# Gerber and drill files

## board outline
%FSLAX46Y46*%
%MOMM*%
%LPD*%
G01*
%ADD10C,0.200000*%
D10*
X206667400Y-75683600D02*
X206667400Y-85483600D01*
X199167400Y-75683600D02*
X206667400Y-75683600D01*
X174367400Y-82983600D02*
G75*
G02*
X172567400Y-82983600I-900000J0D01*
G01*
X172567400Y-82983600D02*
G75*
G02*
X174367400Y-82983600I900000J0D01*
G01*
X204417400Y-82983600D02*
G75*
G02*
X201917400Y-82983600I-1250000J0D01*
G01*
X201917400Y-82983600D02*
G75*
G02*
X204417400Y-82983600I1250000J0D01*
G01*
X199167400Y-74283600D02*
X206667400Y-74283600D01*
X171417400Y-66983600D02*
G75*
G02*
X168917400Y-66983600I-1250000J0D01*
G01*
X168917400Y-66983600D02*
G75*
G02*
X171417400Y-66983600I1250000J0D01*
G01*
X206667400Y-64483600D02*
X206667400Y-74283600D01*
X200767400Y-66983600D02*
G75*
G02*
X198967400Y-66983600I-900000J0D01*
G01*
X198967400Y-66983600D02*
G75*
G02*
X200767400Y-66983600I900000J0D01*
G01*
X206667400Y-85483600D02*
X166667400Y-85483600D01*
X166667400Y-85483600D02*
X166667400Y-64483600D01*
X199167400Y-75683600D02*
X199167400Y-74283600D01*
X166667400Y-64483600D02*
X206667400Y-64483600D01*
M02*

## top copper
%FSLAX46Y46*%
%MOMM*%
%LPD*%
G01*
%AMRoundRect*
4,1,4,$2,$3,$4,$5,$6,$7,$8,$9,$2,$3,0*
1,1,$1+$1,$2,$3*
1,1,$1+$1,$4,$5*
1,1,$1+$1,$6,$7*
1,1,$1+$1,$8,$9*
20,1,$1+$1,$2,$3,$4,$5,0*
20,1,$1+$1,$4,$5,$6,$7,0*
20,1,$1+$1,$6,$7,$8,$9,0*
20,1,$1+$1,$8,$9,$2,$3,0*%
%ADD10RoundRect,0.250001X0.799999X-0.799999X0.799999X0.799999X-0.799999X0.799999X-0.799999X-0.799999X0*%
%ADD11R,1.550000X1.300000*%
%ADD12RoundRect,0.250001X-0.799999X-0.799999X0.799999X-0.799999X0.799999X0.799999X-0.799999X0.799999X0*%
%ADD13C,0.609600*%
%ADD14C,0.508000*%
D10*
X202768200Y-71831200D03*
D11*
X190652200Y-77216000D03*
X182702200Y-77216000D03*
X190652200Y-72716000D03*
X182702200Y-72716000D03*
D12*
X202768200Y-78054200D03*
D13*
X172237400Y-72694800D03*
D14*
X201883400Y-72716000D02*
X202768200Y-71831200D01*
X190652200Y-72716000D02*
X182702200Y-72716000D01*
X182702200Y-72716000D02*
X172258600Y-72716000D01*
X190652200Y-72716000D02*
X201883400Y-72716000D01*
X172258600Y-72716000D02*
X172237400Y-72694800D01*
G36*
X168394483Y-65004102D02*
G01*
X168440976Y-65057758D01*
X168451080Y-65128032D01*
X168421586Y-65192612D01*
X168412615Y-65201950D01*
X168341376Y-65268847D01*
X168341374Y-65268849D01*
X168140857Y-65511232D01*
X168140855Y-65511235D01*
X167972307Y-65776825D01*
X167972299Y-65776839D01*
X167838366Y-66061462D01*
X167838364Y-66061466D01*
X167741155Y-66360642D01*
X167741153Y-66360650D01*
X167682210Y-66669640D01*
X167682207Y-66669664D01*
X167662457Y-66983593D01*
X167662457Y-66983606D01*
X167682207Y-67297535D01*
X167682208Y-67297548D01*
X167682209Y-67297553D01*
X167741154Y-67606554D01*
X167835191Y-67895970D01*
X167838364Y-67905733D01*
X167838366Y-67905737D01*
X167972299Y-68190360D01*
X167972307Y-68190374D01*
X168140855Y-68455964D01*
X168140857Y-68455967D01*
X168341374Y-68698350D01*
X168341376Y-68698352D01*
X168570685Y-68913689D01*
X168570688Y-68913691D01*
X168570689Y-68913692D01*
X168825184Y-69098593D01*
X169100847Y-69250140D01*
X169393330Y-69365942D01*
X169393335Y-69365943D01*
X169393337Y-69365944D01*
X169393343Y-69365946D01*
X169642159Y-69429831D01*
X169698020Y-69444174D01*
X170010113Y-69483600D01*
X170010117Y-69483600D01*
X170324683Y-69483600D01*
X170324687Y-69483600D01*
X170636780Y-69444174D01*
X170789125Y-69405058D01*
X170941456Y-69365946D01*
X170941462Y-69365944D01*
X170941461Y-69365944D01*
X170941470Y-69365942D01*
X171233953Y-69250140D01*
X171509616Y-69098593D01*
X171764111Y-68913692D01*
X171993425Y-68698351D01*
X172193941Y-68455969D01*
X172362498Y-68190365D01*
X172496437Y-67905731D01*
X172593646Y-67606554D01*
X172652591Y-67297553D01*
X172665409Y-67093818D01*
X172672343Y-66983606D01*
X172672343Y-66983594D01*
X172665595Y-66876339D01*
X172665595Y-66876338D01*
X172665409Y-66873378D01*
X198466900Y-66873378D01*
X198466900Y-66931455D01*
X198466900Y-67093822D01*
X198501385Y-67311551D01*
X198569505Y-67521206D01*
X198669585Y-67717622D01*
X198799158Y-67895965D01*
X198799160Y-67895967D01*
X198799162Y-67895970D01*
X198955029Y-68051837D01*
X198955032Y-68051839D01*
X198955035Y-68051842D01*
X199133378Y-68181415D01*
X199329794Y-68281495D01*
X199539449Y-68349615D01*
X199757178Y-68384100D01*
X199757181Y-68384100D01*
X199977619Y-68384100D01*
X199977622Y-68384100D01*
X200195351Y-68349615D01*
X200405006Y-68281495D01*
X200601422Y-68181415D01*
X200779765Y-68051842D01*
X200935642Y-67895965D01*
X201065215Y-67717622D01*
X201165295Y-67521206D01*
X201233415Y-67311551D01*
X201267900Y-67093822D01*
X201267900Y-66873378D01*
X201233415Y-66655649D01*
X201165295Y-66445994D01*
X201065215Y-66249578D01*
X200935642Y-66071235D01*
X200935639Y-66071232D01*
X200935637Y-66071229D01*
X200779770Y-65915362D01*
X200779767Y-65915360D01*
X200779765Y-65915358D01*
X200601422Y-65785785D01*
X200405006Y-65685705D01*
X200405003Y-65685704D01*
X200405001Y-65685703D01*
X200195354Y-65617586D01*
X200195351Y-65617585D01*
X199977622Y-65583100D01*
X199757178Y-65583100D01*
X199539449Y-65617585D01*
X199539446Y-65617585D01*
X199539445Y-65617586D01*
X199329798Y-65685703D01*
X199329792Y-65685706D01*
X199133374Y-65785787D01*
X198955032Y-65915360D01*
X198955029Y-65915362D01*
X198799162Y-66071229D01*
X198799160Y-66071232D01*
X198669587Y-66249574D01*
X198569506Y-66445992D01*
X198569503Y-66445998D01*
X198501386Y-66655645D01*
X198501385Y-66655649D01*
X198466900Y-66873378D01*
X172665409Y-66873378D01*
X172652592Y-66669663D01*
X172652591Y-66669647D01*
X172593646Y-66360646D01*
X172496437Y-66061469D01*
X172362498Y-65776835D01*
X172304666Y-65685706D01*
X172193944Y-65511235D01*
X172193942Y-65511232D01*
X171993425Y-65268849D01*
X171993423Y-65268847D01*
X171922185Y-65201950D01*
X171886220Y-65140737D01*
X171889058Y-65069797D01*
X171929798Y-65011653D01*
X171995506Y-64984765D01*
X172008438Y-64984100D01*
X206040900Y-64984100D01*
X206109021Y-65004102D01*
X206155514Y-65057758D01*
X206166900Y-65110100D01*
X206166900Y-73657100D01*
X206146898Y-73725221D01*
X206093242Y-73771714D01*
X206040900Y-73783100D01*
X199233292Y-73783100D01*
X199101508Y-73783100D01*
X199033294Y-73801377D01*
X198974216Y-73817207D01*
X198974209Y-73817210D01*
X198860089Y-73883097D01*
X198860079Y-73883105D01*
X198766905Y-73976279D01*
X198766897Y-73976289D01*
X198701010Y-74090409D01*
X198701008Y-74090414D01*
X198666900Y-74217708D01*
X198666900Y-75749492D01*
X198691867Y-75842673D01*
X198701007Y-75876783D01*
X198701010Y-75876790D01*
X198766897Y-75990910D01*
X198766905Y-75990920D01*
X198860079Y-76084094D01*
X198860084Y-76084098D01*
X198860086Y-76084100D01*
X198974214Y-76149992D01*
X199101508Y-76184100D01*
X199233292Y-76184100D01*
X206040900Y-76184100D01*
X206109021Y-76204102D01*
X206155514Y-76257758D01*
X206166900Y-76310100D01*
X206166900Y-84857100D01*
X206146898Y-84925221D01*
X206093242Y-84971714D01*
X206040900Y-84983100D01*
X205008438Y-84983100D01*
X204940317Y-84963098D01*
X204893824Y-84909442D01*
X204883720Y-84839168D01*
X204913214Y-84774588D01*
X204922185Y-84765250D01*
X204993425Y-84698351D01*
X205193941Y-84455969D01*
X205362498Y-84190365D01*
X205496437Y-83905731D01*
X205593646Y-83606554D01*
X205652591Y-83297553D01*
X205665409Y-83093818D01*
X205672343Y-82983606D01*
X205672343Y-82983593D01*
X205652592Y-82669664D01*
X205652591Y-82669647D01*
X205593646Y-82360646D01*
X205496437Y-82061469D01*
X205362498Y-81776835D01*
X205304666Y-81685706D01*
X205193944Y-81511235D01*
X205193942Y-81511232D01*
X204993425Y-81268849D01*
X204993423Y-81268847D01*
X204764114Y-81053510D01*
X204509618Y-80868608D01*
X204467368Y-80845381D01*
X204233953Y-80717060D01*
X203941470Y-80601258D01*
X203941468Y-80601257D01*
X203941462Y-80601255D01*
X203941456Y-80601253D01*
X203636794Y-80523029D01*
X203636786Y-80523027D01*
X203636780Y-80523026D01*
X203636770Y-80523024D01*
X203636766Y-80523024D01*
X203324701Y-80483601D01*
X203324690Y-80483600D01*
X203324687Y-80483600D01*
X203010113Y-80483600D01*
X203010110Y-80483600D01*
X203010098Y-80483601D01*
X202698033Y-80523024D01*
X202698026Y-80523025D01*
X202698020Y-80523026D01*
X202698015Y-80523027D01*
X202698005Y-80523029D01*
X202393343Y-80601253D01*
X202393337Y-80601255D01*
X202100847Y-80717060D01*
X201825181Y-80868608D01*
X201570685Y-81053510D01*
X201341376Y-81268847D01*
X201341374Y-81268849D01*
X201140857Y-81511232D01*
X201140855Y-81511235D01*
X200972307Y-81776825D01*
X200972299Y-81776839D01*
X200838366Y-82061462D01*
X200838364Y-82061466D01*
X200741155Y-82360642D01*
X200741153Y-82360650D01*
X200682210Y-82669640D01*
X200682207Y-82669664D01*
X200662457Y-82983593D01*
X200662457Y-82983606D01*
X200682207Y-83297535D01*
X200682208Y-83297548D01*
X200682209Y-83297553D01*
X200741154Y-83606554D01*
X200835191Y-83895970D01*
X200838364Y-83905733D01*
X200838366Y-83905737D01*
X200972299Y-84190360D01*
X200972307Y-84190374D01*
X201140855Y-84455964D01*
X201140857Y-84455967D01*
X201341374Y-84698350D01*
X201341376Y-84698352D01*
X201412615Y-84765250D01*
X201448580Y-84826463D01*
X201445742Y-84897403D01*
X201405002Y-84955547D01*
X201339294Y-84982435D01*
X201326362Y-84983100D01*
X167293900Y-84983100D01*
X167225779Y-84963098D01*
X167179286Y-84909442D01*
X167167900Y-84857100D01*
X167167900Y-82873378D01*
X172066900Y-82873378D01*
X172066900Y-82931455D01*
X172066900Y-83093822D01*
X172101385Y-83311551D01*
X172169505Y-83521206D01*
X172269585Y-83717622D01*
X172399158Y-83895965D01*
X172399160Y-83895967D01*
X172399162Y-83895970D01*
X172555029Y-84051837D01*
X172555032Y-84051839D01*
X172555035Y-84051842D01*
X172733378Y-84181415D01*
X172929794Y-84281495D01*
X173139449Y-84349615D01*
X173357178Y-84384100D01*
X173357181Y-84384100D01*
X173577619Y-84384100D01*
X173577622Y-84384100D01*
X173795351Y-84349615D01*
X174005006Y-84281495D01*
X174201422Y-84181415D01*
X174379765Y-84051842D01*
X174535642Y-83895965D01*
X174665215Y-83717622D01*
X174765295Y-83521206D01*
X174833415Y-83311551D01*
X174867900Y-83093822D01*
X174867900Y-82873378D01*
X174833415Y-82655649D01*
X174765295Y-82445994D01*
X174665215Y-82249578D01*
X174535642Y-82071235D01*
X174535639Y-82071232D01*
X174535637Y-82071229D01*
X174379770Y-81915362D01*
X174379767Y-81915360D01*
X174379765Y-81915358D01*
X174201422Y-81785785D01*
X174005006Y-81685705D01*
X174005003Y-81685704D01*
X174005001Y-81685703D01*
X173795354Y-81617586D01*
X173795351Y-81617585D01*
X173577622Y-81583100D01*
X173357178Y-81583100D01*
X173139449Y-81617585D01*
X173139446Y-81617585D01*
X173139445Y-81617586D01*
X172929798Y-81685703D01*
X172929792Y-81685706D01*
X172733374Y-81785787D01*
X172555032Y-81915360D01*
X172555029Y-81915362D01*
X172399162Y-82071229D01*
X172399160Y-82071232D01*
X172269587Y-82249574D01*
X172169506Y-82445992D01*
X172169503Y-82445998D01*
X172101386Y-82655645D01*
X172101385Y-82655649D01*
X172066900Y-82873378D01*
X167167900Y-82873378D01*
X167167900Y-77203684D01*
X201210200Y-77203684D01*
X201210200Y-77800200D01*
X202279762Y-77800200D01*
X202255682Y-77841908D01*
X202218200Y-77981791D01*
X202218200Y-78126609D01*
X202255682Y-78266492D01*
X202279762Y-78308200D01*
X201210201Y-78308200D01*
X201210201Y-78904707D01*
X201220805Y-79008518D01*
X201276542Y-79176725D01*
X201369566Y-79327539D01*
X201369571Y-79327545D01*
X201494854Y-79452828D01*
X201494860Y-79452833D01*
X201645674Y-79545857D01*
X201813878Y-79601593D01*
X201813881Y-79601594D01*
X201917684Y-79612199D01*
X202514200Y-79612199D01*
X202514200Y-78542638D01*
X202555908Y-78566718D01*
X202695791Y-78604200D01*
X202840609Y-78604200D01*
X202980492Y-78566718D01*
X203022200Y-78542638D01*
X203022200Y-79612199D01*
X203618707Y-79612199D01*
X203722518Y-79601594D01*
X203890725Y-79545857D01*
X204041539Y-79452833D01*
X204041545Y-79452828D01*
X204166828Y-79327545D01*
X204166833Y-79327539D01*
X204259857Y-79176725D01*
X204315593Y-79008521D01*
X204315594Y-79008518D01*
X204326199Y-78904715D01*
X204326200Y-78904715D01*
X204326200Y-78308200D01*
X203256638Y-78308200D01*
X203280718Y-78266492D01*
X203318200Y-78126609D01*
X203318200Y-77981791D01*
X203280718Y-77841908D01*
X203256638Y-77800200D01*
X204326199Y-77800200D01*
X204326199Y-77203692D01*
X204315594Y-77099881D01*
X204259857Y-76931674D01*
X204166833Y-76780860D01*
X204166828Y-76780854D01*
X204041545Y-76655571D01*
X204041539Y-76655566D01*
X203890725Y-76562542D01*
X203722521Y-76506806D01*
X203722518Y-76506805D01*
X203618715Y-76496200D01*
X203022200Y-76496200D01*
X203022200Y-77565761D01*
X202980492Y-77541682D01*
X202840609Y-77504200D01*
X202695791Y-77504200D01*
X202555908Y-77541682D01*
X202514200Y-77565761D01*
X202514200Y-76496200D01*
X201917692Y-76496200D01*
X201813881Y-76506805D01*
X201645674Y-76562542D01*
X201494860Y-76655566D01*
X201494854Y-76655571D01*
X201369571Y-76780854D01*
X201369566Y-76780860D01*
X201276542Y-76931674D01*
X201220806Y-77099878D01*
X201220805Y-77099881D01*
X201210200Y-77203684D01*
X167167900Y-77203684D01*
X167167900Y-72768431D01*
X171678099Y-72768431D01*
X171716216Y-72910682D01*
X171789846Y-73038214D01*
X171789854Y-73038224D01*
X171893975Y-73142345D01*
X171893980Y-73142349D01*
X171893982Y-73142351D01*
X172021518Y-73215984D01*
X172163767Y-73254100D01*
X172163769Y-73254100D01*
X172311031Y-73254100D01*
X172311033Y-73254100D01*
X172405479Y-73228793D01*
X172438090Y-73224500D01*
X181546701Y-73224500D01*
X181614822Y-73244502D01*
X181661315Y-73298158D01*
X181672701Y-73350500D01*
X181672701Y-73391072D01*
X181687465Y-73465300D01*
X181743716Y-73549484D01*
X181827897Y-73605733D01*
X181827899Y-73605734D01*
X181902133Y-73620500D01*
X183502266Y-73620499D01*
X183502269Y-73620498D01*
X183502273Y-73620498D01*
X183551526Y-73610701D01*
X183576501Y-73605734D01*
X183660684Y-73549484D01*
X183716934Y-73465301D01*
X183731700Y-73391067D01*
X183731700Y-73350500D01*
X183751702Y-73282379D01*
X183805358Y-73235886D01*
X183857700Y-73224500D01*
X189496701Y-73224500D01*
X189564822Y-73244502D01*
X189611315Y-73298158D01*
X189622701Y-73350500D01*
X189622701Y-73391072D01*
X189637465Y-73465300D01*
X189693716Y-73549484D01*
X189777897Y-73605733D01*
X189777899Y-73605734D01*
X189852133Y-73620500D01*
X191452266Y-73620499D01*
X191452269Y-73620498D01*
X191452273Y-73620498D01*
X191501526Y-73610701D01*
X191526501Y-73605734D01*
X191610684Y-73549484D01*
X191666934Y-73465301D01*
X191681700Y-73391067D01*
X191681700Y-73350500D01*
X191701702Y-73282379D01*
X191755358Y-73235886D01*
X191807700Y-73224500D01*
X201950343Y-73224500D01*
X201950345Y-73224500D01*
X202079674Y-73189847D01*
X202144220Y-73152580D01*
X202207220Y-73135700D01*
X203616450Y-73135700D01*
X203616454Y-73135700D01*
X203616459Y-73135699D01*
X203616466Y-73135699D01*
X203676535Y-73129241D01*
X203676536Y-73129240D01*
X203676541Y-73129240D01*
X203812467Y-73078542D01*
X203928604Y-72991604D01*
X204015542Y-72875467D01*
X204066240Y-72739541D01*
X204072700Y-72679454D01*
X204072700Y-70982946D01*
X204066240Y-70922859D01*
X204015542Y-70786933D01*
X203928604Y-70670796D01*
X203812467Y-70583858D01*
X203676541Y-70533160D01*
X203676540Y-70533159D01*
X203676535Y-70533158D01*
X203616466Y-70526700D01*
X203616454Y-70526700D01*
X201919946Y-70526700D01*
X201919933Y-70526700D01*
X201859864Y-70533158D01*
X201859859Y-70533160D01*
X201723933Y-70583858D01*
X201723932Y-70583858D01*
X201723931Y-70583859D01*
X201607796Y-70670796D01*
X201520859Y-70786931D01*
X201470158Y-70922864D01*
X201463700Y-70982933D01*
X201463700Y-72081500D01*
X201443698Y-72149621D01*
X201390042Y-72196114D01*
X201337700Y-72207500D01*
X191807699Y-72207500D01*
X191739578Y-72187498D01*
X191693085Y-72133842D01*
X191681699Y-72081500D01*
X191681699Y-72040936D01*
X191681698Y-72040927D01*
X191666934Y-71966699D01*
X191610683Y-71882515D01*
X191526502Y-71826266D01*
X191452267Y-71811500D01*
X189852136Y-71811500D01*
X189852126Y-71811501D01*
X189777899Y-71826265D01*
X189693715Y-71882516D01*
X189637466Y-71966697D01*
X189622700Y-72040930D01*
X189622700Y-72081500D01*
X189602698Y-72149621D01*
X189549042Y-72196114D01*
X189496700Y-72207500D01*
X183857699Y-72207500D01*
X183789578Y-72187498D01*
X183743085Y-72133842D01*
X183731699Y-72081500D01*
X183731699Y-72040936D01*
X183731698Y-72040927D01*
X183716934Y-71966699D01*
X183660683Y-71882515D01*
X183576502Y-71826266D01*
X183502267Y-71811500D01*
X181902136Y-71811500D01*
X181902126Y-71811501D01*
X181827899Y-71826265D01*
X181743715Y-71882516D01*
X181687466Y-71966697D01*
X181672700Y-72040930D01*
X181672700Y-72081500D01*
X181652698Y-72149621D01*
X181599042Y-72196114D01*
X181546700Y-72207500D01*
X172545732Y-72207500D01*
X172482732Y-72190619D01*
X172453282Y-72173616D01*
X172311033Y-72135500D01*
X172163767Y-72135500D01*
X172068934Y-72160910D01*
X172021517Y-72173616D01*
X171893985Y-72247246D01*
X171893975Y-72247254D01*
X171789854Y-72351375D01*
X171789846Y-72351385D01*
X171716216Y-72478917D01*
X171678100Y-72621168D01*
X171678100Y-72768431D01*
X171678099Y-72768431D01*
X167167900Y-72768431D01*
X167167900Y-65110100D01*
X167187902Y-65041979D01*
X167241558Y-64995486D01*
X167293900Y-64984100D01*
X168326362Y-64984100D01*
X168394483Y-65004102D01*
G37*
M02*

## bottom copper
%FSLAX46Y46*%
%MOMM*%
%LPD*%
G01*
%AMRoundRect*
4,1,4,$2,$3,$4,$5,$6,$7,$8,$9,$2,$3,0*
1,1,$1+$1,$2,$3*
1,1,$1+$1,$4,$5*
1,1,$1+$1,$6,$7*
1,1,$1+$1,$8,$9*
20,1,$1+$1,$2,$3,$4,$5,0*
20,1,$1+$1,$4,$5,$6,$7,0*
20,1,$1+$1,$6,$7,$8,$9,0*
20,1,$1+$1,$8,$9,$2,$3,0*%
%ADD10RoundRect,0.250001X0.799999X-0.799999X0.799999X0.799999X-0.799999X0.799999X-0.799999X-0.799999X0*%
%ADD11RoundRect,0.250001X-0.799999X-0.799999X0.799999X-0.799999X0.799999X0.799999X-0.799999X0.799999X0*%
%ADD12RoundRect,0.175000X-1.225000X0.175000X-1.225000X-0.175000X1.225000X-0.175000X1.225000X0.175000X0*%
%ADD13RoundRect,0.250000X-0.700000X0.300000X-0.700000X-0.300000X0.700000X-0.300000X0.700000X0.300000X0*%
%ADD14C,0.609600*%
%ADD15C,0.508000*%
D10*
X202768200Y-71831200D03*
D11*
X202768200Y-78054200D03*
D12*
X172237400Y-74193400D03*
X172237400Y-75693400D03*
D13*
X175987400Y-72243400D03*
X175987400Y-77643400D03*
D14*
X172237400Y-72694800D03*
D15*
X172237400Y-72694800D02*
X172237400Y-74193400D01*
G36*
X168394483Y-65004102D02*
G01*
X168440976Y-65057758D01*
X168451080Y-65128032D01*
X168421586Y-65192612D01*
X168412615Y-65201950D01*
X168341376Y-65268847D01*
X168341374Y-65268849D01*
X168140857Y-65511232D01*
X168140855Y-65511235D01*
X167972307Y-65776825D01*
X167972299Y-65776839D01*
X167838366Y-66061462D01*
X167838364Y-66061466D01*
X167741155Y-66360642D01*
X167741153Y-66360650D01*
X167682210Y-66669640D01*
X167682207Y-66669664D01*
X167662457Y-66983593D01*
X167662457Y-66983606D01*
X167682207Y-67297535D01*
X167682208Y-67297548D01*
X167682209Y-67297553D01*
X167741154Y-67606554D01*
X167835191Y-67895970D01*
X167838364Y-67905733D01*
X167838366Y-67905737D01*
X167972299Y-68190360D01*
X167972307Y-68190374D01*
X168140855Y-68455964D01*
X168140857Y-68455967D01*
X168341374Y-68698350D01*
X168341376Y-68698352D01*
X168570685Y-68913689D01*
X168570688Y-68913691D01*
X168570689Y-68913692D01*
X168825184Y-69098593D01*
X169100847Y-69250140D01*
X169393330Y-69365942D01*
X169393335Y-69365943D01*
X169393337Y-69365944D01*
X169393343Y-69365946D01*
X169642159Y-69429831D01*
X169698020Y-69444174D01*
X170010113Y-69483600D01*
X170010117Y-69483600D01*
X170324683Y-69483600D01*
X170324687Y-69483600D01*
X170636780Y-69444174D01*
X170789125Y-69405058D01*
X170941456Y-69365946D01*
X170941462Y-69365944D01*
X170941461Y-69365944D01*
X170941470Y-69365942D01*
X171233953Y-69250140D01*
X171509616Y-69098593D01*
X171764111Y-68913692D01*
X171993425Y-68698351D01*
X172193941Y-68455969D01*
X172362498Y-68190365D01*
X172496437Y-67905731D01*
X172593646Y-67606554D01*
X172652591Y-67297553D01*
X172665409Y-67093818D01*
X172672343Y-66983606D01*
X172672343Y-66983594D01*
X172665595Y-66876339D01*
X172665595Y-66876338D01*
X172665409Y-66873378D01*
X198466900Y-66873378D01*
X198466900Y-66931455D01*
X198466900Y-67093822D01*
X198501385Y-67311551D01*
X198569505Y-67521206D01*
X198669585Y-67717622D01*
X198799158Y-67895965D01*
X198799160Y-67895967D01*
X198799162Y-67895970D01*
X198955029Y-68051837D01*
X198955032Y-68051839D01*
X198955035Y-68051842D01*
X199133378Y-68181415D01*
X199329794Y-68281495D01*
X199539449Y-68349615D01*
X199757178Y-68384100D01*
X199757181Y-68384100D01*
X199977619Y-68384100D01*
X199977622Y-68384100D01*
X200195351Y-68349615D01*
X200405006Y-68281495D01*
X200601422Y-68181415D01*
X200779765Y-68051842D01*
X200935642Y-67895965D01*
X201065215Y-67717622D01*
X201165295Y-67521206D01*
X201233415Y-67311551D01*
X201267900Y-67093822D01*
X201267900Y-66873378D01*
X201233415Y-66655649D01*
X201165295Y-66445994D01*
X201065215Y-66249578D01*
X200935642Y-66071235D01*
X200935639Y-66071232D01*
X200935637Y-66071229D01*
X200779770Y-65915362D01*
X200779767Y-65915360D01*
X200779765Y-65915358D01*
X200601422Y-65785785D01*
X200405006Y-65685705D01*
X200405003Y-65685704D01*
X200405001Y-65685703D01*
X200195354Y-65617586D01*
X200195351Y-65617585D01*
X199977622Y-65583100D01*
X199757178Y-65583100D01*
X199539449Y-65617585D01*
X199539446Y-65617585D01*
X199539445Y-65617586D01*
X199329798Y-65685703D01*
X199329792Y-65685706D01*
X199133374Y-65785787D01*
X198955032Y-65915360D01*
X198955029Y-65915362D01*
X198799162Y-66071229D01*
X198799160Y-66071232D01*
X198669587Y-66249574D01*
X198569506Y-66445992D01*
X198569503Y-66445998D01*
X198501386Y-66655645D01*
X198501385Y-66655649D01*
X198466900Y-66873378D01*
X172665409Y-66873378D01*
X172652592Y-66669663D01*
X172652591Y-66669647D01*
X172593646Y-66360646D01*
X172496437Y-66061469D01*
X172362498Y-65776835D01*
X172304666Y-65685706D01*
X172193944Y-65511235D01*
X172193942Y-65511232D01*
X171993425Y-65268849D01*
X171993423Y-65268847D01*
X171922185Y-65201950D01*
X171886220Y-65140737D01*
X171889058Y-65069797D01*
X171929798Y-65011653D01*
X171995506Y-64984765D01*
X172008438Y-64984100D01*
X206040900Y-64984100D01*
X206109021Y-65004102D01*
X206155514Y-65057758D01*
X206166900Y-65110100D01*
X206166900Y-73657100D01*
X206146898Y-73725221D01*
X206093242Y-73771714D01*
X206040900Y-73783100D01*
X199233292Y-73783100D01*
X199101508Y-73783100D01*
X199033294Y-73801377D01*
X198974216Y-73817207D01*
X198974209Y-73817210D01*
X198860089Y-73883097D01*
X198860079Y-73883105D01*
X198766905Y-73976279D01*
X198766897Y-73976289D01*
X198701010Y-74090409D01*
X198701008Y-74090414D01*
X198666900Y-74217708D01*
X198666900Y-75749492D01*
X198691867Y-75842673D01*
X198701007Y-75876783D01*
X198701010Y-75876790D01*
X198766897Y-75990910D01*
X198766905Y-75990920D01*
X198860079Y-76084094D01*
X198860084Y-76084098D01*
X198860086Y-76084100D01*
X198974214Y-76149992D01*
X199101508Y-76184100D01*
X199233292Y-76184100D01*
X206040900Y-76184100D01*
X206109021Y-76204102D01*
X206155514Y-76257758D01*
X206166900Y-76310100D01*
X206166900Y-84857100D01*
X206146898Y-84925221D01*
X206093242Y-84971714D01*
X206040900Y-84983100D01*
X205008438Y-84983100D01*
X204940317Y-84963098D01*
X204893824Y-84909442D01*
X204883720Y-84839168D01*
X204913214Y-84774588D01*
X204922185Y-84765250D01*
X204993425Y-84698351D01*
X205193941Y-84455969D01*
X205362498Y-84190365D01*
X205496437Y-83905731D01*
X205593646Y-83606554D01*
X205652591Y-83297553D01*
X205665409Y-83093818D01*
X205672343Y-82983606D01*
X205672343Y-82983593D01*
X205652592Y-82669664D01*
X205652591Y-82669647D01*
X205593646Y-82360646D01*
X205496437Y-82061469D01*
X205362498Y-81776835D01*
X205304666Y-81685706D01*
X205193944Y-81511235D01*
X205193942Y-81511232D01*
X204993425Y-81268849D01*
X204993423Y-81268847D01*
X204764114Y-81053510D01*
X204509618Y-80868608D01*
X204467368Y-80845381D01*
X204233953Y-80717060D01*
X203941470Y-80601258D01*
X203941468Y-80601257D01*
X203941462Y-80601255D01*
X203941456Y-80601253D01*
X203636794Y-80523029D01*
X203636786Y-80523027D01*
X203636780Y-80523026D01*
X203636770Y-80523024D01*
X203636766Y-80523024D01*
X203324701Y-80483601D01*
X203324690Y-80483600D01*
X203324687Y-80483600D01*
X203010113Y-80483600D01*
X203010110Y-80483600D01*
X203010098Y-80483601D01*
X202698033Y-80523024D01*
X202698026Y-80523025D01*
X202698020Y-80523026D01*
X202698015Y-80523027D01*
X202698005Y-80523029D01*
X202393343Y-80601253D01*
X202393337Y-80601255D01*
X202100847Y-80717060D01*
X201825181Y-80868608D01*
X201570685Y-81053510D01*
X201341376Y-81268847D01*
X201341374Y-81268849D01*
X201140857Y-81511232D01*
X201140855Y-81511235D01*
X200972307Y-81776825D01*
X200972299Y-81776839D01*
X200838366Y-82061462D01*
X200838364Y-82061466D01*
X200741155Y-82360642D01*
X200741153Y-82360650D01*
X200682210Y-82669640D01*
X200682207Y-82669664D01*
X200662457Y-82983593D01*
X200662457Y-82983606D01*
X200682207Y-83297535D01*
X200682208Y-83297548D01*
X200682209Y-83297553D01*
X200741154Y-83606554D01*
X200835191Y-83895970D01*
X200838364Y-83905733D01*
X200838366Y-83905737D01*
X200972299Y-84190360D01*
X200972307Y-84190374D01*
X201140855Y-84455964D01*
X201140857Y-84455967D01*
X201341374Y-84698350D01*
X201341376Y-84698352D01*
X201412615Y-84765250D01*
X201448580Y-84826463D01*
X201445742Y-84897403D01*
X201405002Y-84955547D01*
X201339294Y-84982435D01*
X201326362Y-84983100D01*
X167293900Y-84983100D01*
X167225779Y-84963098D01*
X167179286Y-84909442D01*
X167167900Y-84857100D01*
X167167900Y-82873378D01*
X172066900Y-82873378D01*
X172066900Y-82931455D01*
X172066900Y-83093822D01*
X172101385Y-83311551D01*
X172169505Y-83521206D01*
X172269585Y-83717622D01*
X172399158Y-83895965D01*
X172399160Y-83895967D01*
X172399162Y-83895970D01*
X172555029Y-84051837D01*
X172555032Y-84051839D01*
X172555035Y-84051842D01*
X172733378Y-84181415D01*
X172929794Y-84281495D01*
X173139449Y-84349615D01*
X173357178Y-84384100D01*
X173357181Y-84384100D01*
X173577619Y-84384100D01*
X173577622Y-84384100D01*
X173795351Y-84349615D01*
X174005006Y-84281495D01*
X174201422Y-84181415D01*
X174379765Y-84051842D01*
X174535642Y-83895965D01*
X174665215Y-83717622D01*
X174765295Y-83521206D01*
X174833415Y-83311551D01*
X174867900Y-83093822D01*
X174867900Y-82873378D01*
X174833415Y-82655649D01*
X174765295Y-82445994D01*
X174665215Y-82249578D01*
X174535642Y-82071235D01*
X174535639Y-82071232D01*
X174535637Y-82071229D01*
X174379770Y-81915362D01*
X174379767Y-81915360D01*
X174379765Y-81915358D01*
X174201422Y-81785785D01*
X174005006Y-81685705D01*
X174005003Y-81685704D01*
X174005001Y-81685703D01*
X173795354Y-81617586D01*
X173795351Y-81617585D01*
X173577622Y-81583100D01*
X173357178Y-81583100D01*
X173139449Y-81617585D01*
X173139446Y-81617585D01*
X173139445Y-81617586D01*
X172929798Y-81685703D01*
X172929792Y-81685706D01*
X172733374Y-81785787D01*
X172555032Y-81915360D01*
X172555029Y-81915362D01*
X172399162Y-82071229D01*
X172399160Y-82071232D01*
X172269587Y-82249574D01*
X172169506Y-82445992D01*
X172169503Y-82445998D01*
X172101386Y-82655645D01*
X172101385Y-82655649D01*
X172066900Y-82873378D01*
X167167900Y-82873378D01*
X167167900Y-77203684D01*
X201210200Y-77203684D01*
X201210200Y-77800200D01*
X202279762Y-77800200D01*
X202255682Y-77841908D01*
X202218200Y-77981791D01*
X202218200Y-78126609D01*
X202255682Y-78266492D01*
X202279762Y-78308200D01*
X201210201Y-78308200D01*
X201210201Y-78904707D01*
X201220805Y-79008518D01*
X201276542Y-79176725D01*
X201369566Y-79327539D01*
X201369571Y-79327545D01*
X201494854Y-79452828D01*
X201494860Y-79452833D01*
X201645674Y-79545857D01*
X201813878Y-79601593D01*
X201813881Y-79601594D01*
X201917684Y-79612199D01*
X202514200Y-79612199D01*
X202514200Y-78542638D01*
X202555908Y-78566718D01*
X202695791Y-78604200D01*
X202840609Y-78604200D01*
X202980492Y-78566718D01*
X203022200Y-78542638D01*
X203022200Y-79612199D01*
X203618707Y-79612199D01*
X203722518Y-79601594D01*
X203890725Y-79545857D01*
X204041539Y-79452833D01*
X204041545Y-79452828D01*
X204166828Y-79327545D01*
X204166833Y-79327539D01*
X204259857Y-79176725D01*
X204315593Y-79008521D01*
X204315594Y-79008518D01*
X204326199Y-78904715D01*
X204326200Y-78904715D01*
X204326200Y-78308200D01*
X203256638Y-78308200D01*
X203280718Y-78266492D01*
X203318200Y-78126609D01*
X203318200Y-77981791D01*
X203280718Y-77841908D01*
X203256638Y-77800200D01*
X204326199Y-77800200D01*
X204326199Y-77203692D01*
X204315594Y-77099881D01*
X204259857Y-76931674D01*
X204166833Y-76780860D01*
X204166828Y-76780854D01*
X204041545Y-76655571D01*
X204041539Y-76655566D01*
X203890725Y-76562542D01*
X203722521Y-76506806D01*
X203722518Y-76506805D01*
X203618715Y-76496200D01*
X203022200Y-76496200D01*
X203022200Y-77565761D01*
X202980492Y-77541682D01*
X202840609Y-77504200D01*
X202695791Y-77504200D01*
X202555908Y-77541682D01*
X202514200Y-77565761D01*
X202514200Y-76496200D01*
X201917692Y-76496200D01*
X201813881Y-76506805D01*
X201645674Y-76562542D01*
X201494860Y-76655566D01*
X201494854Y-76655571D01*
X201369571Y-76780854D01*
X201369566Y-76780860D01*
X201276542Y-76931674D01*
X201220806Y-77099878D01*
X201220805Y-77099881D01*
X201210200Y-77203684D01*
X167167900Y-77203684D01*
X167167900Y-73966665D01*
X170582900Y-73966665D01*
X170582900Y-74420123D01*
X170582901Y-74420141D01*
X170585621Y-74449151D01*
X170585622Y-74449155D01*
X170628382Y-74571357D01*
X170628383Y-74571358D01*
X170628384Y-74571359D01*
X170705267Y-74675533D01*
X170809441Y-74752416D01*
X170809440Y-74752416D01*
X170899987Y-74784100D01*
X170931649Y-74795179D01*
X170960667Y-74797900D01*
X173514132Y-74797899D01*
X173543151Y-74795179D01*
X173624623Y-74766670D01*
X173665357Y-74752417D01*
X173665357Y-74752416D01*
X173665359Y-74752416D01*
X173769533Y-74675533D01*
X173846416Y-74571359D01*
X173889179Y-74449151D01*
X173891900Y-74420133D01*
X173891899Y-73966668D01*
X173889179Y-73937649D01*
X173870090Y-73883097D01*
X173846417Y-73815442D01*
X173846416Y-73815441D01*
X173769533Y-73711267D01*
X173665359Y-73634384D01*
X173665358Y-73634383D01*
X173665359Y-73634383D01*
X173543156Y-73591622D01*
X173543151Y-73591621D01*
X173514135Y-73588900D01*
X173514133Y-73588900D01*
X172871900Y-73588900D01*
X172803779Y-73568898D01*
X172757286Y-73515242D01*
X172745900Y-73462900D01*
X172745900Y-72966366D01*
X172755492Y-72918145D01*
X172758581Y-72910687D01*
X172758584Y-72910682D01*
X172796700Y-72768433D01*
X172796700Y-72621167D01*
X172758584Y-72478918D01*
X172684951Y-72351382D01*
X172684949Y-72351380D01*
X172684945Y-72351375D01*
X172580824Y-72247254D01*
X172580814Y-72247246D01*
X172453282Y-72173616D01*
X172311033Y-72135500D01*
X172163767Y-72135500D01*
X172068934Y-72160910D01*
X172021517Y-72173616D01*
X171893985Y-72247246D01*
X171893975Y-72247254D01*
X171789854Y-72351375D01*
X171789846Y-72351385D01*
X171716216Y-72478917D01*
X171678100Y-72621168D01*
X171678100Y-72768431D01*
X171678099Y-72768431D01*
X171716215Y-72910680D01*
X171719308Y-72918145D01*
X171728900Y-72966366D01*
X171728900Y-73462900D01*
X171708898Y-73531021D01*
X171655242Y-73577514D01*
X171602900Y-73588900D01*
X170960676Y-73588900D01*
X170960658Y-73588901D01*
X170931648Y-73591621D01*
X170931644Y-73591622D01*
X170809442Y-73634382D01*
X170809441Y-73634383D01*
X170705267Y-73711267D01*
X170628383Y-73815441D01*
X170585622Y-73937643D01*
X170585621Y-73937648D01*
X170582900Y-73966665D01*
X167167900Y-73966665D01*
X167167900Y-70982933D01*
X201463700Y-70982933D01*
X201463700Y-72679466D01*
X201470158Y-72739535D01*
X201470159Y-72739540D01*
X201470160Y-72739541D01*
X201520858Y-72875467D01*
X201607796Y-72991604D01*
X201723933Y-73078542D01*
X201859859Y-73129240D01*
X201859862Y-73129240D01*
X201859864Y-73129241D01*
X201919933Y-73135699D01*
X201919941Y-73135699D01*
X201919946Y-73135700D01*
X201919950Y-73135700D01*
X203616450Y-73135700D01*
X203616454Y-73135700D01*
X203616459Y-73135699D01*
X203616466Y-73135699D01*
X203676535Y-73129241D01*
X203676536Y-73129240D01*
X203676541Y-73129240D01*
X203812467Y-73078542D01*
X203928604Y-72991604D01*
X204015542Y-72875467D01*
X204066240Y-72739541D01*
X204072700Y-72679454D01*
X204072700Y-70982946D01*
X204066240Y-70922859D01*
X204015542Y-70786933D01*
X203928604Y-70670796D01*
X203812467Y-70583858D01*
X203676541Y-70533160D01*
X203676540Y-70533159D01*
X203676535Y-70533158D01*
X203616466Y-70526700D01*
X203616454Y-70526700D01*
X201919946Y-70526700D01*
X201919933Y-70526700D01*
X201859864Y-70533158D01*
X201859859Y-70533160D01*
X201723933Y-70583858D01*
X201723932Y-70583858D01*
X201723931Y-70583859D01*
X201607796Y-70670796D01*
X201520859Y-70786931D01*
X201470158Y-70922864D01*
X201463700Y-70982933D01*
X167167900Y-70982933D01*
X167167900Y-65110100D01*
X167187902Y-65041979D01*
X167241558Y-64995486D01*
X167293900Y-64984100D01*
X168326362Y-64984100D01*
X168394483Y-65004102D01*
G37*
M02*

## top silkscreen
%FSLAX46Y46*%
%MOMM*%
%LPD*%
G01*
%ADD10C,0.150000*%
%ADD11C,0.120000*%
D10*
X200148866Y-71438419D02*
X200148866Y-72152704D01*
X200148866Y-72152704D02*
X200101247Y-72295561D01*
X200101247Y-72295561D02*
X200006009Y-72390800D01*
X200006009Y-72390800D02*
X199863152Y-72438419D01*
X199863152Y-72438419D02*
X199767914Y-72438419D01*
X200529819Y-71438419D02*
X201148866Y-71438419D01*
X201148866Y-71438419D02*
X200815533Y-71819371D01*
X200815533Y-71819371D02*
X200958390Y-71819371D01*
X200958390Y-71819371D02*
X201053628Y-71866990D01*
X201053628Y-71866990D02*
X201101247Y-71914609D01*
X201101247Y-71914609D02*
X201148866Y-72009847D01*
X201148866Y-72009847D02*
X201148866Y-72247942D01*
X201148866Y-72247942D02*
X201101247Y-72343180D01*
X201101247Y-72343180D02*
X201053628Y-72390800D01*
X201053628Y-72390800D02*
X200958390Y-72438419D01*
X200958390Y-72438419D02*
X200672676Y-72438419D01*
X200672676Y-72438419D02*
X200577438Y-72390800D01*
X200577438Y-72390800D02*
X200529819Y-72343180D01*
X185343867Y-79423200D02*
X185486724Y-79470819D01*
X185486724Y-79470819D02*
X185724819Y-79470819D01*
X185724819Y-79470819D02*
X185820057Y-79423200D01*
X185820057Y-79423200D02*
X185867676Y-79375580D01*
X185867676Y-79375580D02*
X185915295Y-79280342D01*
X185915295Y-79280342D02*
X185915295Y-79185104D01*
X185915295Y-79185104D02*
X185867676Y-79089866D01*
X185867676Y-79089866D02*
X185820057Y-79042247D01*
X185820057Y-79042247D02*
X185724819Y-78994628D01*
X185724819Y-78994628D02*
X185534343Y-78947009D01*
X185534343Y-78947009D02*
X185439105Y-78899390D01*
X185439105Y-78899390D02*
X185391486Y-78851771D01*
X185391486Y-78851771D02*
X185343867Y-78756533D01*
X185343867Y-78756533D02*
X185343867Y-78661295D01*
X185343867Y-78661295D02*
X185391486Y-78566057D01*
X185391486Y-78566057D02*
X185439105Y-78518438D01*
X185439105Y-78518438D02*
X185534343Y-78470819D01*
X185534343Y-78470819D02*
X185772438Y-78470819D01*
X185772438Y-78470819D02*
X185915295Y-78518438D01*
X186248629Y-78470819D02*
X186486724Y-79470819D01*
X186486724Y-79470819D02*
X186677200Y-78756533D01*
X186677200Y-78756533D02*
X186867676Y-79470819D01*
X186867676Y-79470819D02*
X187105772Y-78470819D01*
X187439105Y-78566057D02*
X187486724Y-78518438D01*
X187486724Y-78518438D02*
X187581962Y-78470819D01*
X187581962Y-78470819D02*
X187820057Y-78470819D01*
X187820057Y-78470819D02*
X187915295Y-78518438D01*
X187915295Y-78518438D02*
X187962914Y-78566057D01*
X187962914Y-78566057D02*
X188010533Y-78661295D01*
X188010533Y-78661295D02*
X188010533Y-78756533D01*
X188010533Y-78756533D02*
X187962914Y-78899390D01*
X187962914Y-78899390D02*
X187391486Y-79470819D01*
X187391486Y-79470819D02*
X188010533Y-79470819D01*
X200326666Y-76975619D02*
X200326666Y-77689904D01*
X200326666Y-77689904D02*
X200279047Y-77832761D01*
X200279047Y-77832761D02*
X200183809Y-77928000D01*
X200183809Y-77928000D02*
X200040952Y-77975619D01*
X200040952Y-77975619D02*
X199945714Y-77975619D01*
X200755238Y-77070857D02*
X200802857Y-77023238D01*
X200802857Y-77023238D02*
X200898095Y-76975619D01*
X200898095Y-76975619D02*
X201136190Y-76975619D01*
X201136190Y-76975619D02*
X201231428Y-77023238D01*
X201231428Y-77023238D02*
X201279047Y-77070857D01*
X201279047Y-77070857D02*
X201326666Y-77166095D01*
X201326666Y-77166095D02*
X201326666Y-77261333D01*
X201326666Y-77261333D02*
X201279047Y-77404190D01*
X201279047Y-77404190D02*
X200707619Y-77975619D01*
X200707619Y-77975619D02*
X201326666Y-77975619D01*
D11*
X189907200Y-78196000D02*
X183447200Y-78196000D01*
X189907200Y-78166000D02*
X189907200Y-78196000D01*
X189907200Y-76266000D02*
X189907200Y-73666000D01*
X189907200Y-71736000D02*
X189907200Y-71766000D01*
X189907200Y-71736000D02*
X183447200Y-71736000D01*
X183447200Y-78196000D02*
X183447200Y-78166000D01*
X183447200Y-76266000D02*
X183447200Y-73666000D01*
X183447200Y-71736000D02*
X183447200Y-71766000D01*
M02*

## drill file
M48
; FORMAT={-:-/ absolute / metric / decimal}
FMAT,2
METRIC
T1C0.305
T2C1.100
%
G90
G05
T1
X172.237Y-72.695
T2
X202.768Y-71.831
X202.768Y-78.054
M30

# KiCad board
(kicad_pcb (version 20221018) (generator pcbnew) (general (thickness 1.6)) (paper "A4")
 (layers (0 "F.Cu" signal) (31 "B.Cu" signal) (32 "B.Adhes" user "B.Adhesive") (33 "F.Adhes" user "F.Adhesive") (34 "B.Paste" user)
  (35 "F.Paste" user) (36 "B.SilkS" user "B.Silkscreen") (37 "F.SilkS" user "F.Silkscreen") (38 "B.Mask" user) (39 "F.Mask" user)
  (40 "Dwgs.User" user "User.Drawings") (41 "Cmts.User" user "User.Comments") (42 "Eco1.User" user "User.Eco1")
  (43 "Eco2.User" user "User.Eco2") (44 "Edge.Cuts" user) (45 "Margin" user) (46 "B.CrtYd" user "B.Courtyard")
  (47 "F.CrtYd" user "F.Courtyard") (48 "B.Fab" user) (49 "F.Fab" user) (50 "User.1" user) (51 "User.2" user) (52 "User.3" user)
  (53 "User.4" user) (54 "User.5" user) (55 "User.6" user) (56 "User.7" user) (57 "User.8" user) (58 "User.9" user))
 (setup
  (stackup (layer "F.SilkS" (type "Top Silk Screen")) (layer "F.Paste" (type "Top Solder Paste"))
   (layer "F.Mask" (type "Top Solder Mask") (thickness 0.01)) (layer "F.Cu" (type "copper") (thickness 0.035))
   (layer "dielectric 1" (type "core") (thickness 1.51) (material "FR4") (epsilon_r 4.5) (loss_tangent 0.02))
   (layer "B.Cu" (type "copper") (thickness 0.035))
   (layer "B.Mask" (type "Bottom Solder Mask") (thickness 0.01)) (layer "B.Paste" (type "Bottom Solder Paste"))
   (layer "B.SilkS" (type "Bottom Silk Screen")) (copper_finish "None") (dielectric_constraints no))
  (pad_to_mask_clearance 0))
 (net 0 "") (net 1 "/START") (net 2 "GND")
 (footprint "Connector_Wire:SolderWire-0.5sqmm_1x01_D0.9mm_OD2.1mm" (layer "F.Cu") (at 202.7682 71.8312 90)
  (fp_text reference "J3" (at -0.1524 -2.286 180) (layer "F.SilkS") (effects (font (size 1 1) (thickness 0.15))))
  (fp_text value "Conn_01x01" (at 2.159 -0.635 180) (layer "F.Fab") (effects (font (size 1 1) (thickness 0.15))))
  (pad "1" thru_hole roundrect (at 0 0 90) (size 2.1 2.1) (drill 1.1) (layers "*.Cu" "*.Mask") (roundrect_rratio 0.119048) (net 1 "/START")))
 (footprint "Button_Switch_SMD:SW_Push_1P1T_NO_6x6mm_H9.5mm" (layer "F.Cu") (at 186.6772 74.966 180)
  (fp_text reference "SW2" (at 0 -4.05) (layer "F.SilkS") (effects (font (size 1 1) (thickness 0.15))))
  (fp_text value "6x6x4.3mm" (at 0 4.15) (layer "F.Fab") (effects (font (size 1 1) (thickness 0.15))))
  (fp_line (start -3.23 -3.23) (end 3.23 -3.23) (stroke (width 0.12) (type solid)) (layer "F.SilkS"))
  (fp_line (start -3.23 -3.2) (end -3.23 -3.23) (stroke (width 0.12) (type solid)) (layer "F.SilkS"))
  (fp_line (start -3.23 -1.3) (end -3.23 1.3) (stroke (width 0.12) (type solid)) (layer "F.SilkS"))
  (fp_line (start -3.23 3.23) (end -3.23 3.2) (stroke (width 0.12) (type solid)) (layer "F.SilkS"))
  (fp_line (start -3.23 3.23) (end 3.23 3.23) (stroke (width 0.12) (type solid)) (layer "F.SilkS"))
  (fp_line (start 3.23 -3.23) (end 3.23 -3.2) (stroke (width 0.12) (type solid)) (layer "F.SilkS"))
  (fp_line (start 3.23 -1.3) (end 3.23 1.3) (stroke (width 0.12) (type solid)) (layer "F.SilkS"))
  (fp_line (start 3.23 3.23) (end 3.23 3.2) (stroke (width 0.12) (type solid)) (layer "F.SilkS"))
  (pad "1" smd rect (at -3.975 -2.25 180) (size 1.55 1.3) (layers "F.Cu" "F.Paste" "F.Mask") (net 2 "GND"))
  (pad "1" smd rect (at 3.975 -2.25 180) (size 1.55 1.3) (layers "F.Cu" "F.Paste" "F.Mask") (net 2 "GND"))
  (pad "2" smd rect (at -3.975 2.25 180) (size 1.55 1.3) (layers "F.Cu" "F.Paste" "F.Mask") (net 1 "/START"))
  (pad "2" smd rect (at 3.975 2.25 180) (size 1.55 1.3) (layers "F.Cu" "F.Paste" "F.Mask") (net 1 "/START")))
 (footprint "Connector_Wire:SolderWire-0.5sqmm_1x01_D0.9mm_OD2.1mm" (layer "F.Cu") (at 202.7682 78.0542)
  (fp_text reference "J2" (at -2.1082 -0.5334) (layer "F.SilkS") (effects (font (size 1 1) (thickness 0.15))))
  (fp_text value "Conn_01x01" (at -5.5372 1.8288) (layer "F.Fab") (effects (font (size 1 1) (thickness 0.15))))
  (pad "1" thru_hole roundrect (at 0 0) (size 2.1 2.1) (drill 1.1) (layers "*.Cu" "*.Mask") (roundrect_rratio 0.119048) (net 2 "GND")))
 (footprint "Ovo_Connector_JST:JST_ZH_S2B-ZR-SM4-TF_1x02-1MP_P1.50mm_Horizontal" (layer "B.Cu") (at 173.8874 74.9434 -90)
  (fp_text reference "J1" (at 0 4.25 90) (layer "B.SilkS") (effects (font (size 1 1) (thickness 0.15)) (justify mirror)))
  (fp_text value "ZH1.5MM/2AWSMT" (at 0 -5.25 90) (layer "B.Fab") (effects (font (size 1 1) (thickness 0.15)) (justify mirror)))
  (pad "1" smd roundrect (at -0.75 1.65 270) (size 0.7 2.8) (layers "B.Cu" "B.Paste" "B.Mask") (roundrect_rratio 0.25) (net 1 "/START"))
  (pad "2" smd roundrect (at 0.75 1.65 270) (size 0.7 2.8) (layers "B.Cu" "B.Paste" "B.Mask") (roundrect_rratio 0.25) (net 2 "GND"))
  (pad "MP" smd roundrect (at -2.7 -2.1 270) (size 1.1 1.9) (layers "B.Cu" "B.Paste" "B.Mask") (roundrect_rratio 0.227273) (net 2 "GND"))
  (pad "MP" smd roundrect (at 2.7 -2.1 270) (size 1.1 1.9) (layers "B.Cu" "B.Paste" "B.Mask") (roundrect_rratio 0.227273) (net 2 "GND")))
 (gr_line (start 206.6674 75.6836) (end 206.6674 85.4836) (stroke (width 0.2) (type solid)) (layer "Edge.Cuts"))
 (gr_line (start 199.1674 75.6836) (end 206.6674 75.6836) (stroke (width 0.2) (type solid)) (layer "Edge.Cuts"))
 (gr_circle (center 173.4674 82.9836) (end 174.3674 82.9836) (stroke (width 0.2) (type solid)) (fill none) (layer "Edge.Cuts"))
 (gr_circle (center 203.1674 82.9836) (end 204.4174 82.9836) (stroke (width 0.2) (type solid)) (fill none) (layer "Edge.Cuts"))
 (gr_line (start 199.1674 74.2836) (end 206.6674 74.2836) (stroke (width 0.2) (type solid)) (layer "Edge.Cuts"))
 (gr_circle (center 170.1674 66.9836) (end 171.4174 66.9836) (stroke (width 0.2) (type solid)) (fill none) (layer "Edge.Cuts"))
 (gr_line (start 206.6674 64.4836) (end 206.6674 74.2836) (stroke (width 0.2) (type solid)) (layer "Edge.Cuts"))
 (gr_circle (center 199.8674 66.9836) (end 200.7674 66.9836) (stroke (width 0.2) (type solid)) (fill none) (layer "Edge.Cuts"))
 (gr_line (start 206.6674 85.4836) (end 166.6674 85.4836) (stroke (width 0.2) (type solid)) (layer "Edge.Cuts"))
 (gr_line (start 166.6674 85.4836) (end 166.6674 64.4836) (stroke (width 0.2) (type solid)) (layer "Edge.Cuts"))
 (gr_line (start 199.1674 75.6836) (end 199.1674 74.2836) (stroke (width 0.2) (type solid)) (layer "Edge.Cuts"))
 (gr_line (start 166.6674 64.4836) (end 206.6674 64.4836) (stroke (width 0.2) (type solid)) (layer "Edge.Cuts"))
 (segment (start 201.8834 72.716) (end 202.7682 71.8312) (width 0.508) (layer "F.Cu") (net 1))
 (segment (start 190.6522 72.716) (end 182.7022 72.716) (width 0.508) (layer "F.Cu") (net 1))
 (segment (start 182.7022 72.716) (end 172.2586 72.716) (width 0.508) (layer "F.Cu") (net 1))
 (segment (start 190.6522 72.716) (end 201.8834 72.716) (width 0.508) (layer "F.Cu") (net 1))
 (segment (start 172.2586 72.716) (end 172.2374 72.6948) (width 0.508) (layer "F.Cu") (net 1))
 (via (at 172.2374 72.6948) (size 0.6096) (drill 0.3048) (layers "F.Cu" "B.Cu") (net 1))
 (segment (start 172.2374 72.6948) (end 172.2374 74.1934) (width 0.508) (layer "B.Cu") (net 1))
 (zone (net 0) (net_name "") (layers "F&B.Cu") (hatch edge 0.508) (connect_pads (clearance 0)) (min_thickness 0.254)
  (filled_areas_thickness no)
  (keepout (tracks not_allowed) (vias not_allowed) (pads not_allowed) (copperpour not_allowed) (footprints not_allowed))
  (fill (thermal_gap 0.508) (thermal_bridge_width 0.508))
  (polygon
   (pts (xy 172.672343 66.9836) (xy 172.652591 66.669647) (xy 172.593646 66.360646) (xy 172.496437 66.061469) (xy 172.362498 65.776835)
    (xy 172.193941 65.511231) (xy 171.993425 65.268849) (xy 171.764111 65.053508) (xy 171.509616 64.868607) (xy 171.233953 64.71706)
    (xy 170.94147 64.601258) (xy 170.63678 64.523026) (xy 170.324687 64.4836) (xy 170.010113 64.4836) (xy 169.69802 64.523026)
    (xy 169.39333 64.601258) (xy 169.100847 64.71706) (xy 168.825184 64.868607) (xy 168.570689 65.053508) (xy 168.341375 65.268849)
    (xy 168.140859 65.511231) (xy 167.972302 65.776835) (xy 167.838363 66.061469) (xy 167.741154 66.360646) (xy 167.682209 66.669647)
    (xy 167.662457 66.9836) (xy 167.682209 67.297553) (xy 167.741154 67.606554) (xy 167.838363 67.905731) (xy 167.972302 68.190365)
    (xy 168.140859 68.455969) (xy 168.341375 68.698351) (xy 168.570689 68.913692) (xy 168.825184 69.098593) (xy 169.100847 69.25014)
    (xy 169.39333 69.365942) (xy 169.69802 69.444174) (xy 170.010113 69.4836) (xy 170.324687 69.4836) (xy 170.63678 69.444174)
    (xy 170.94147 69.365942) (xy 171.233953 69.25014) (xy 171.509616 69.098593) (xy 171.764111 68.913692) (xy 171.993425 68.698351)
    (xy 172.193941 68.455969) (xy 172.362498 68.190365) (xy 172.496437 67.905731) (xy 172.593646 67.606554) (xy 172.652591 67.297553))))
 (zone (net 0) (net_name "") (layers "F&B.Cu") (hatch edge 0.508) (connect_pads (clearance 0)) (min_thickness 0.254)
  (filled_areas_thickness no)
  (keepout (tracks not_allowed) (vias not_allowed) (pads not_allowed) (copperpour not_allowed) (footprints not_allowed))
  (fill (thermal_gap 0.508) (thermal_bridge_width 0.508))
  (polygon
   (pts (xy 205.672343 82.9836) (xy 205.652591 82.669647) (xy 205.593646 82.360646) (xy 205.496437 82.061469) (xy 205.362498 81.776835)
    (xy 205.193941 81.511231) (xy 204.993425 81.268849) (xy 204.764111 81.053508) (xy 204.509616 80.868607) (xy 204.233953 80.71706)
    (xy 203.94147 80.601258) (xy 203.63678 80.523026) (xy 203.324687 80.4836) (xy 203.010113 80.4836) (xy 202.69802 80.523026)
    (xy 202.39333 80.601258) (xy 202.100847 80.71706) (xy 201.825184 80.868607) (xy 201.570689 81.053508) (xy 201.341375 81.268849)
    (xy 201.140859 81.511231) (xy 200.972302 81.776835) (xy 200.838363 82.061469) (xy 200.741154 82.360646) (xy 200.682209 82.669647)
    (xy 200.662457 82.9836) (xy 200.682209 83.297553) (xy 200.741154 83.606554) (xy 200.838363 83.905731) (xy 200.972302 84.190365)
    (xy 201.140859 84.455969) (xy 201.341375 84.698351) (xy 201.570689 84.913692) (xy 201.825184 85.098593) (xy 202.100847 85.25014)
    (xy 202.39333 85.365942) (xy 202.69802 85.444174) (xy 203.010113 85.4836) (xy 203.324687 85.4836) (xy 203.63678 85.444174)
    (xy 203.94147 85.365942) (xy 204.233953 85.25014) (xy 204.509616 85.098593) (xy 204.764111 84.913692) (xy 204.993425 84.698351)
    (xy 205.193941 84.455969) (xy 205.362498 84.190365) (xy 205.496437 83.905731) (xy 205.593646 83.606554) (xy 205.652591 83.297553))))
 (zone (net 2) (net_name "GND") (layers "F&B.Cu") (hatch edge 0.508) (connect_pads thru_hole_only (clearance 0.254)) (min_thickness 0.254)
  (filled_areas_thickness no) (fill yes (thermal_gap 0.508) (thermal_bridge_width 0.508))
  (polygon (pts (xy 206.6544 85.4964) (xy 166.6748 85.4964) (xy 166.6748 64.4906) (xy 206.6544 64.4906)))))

